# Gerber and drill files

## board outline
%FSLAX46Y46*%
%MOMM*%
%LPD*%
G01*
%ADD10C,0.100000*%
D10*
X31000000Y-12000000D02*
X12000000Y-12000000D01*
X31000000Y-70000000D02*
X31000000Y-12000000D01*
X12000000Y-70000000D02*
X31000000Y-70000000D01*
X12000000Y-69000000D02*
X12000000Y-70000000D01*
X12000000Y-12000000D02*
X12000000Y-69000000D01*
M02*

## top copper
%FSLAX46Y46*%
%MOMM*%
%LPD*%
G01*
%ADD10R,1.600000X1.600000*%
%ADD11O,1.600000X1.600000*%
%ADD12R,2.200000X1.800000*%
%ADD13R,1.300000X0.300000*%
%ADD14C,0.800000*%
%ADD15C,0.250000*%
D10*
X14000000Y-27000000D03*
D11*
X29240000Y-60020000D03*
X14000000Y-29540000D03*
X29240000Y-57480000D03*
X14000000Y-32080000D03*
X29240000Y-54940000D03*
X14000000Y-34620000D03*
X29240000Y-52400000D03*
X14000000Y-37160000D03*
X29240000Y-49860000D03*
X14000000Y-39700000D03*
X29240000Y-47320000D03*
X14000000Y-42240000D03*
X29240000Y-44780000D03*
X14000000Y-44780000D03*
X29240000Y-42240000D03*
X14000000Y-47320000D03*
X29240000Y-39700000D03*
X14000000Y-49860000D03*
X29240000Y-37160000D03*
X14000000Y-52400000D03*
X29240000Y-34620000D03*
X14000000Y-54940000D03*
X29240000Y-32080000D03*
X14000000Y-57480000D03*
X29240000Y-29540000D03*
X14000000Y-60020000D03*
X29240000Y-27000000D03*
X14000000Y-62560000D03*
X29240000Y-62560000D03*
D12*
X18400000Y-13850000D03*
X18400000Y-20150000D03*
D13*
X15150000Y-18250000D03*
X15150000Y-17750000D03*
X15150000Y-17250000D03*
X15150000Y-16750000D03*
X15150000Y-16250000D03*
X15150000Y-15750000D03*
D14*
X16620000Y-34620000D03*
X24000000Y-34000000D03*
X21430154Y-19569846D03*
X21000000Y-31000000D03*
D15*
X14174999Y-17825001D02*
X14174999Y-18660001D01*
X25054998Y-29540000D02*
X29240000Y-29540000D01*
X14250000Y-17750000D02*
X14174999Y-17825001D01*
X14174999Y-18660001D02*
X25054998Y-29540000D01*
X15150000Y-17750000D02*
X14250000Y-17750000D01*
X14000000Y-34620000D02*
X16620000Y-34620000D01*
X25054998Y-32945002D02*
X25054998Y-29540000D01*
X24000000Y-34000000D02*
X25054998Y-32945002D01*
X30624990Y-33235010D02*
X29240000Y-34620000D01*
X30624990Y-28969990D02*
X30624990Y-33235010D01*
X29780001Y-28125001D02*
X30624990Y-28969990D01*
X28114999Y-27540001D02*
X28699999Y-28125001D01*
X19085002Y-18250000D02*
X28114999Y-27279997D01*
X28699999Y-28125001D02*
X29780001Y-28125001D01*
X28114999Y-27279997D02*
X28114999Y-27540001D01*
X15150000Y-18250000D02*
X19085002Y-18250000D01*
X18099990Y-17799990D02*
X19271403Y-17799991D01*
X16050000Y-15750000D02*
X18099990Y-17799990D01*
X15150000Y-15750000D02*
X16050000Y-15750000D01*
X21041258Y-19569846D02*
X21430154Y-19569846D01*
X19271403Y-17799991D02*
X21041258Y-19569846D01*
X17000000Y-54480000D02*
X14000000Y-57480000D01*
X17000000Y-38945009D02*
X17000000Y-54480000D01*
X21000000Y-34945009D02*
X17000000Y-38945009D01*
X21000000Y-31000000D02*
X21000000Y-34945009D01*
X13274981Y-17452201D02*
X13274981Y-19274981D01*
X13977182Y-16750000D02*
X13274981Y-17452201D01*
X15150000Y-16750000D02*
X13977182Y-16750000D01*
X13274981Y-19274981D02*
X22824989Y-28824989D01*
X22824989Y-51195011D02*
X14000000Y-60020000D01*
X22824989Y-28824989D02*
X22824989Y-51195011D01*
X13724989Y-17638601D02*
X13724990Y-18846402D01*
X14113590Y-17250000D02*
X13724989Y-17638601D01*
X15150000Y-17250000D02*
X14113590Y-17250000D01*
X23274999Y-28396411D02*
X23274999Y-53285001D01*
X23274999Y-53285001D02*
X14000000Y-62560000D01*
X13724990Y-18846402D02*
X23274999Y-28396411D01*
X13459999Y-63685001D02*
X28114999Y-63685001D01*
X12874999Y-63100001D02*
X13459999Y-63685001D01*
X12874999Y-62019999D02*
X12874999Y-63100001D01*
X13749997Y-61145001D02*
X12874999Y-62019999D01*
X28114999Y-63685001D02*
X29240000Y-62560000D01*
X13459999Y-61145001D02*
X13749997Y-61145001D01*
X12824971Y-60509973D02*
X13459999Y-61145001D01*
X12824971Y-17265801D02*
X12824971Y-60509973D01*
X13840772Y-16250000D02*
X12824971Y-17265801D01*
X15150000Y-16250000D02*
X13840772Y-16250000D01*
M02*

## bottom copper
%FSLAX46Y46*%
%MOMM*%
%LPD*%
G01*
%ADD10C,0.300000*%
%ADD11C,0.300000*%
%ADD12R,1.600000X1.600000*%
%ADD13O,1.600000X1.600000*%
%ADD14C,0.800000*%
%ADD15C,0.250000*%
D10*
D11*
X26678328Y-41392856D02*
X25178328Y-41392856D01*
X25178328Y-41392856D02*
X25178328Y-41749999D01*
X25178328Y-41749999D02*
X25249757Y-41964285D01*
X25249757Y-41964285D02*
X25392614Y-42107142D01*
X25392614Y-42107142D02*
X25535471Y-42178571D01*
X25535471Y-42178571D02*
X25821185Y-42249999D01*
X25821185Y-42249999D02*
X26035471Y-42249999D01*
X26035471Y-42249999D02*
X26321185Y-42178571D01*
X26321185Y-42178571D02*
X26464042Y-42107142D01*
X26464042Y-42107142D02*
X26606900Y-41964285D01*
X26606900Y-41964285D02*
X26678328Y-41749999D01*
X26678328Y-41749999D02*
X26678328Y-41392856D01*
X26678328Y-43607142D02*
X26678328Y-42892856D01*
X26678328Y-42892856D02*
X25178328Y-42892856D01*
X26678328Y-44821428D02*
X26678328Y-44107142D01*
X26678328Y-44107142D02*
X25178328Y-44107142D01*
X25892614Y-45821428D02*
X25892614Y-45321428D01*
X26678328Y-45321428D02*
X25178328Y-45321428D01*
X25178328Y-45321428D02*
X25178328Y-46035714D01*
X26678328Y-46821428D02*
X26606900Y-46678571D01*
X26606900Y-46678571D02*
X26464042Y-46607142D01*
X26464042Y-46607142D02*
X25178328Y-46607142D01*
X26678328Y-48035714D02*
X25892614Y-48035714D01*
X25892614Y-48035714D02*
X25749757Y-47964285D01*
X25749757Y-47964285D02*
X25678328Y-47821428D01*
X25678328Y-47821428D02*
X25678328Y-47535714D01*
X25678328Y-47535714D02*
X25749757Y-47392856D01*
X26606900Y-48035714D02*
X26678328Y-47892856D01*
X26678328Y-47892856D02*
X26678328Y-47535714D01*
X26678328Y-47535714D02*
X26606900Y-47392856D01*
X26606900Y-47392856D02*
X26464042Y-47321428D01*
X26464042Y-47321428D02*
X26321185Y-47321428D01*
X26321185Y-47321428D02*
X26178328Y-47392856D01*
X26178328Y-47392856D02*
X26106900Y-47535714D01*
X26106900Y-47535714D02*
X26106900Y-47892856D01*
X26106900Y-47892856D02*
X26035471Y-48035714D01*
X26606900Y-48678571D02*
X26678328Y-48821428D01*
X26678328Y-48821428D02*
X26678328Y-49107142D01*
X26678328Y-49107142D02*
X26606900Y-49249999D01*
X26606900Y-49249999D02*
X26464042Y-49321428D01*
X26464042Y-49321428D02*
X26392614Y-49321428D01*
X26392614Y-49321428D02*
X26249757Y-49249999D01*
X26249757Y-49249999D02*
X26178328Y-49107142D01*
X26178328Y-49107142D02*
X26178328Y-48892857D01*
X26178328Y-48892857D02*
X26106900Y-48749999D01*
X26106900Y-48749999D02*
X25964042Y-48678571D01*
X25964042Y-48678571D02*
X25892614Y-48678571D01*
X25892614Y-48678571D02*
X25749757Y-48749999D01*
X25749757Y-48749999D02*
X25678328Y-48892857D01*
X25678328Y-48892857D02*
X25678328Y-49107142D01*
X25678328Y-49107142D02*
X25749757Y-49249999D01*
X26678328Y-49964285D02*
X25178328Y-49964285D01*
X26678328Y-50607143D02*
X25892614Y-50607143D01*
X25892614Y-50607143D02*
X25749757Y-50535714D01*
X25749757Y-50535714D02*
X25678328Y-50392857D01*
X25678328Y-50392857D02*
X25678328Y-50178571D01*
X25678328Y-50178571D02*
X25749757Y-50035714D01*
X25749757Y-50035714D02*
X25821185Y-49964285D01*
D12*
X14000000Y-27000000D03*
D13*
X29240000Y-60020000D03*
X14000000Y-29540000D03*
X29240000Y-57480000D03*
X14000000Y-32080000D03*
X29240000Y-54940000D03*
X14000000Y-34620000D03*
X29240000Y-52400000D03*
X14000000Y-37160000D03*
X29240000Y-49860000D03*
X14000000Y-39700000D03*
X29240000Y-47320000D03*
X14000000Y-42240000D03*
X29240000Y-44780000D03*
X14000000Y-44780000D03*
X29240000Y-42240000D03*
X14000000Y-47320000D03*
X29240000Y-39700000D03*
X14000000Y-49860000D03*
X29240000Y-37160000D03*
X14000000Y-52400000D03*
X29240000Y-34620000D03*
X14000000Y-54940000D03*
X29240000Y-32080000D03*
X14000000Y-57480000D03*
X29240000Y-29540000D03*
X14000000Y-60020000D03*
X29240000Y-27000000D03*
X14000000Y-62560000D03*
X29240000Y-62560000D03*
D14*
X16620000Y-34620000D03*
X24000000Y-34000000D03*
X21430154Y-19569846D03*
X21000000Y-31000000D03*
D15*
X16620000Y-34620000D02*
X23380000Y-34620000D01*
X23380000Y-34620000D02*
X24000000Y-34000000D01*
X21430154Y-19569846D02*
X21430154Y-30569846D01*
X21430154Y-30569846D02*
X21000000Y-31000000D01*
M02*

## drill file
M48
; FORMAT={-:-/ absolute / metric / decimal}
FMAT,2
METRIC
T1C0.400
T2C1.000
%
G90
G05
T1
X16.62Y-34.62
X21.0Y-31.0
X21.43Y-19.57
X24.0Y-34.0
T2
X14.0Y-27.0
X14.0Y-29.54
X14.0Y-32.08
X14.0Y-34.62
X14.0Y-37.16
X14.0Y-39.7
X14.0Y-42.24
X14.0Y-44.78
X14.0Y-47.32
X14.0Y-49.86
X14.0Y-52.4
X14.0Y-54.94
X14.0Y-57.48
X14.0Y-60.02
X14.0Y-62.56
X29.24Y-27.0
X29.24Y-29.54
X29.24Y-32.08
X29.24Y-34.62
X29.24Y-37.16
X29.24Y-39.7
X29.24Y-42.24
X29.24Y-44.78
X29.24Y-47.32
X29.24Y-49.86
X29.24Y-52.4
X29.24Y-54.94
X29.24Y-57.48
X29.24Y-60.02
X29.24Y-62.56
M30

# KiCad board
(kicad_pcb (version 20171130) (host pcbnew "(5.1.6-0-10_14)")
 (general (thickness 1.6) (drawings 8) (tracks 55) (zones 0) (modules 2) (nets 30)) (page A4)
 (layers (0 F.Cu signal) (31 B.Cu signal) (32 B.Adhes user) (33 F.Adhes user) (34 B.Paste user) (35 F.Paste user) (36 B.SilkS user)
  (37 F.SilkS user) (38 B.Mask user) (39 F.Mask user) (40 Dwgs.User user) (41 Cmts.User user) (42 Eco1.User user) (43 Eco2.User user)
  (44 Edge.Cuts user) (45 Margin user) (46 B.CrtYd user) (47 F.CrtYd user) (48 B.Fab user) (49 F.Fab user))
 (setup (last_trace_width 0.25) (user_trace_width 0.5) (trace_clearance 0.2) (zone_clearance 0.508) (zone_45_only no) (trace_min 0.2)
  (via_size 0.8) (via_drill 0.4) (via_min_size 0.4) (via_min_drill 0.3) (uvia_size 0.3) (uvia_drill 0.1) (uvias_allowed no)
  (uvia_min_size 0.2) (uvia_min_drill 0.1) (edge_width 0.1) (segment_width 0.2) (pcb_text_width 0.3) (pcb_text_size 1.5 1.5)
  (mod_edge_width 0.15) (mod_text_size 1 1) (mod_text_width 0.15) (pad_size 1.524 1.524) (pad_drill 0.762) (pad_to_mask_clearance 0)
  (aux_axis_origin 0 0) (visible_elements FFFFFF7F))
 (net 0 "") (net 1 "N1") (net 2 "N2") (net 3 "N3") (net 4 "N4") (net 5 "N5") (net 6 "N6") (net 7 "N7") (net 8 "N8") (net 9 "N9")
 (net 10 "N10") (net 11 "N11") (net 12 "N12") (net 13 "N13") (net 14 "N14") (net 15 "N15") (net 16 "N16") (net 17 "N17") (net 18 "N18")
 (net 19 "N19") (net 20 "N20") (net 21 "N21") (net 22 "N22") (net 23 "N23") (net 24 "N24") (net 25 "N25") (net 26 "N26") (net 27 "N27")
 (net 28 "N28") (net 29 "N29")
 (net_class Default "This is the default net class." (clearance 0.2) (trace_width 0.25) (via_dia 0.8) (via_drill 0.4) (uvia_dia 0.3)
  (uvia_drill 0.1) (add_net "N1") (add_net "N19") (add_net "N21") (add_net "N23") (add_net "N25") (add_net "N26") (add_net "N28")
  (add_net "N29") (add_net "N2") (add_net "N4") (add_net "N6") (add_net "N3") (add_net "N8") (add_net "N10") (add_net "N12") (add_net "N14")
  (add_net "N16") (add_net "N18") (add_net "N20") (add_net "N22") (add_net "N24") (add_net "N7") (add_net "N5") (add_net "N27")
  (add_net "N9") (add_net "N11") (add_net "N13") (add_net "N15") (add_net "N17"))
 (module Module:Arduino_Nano (layer F.Cu) (at 14 27)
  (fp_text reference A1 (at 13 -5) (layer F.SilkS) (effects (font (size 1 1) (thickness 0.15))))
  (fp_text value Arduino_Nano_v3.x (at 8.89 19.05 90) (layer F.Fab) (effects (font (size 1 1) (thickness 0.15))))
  (pad 1 thru_hole rect (at 0 0) (size 1.6 1.6) (drill 1) (layers *.Cu *.Mask) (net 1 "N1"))
  (pad 17 thru_hole oval (at 15.24 33.02) (size 1.6 1.6) (drill 1) (layers *.Cu *.Mask) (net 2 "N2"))
  (pad 2 thru_hole oval (at 0 2.54) (size 1.6 1.6) (drill 1) (layers *.Cu *.Mask) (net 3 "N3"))
  (pad 18 thru_hole oval (at 15.24 30.48) (size 1.6 1.6) (drill 1) (layers *.Cu *.Mask) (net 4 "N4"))
  (pad 3 thru_hole oval (at 0 5.08) (size 1.6 1.6) (drill 1) (layers *.Cu *.Mask) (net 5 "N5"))
  (pad 19 thru_hole oval (at 15.24 27.94) (size 1.6 1.6) (drill 1) (layers *.Cu *.Mask) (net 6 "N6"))
  (pad 4 thru_hole oval (at 0 7.62) (size 1.6 1.6) (drill 1) (layers *.Cu *.Mask) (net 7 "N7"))
  (pad 20 thru_hole oval (at 15.24 25.4) (size 1.6 1.6) (drill 1) (layers *.Cu *.Mask) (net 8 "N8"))
  (pad 5 thru_hole oval (at 0 10.16) (size 1.6 1.6) (drill 1) (layers *.Cu *.Mask) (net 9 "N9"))
  (pad 21 thru_hole oval (at 15.24 22.86) (size 1.6 1.6) (drill 1) (layers *.Cu *.Mask) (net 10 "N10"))
  (pad 6 thru_hole oval (at 0 12.7) (size 1.6 1.6) (drill 1) (layers *.Cu *.Mask) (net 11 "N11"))
  (pad 22 thru_hole oval (at 15.24 20.32) (size 1.6 1.6) (drill 1) (layers *.Cu *.Mask) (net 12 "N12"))
  (pad 7 thru_hole oval (at 0 15.24) (size 1.6 1.6) (drill 1) (layers *.Cu *.Mask) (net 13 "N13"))
  (pad 23 thru_hole oval (at 15.24 17.78) (size 1.6 1.6) (drill 1) (layers *.Cu *.Mask) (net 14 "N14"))
  (pad 8 thru_hole oval (at 0 17.78) (size 1.6 1.6) (drill 1) (layers *.Cu *.Mask) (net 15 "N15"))
  (pad 24 thru_hole oval (at 15.24 15.24) (size 1.6 1.6) (drill 1) (layers *.Cu *.Mask) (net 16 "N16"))
  (pad 9 thru_hole oval (at 0 20.32) (size 1.6 1.6) (drill 1) (layers *.Cu *.Mask) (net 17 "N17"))
  (pad 25 thru_hole oval (at 15.24 12.7) (size 1.6 1.6) (drill 1) (layers *.Cu *.Mask) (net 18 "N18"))
  (pad 10 thru_hole oval (at 0 22.86) (size 1.6 1.6) (drill 1) (layers *.Cu *.Mask) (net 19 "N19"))
  (pad 26 thru_hole oval (at 15.24 10.16) (size 1.6 1.6) (drill 1) (layers *.Cu *.Mask) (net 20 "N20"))
  (pad 11 thru_hole oval (at 0 25.4) (size 1.6 1.6) (drill 1) (layers *.Cu *.Mask) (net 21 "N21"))
  (pad 27 thru_hole oval (at 15.24 7.62) (size 1.6 1.6) (drill 1) (layers *.Cu *.Mask) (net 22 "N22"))
  (pad 12 thru_hole oval (at 0 27.94) (size 1.6 1.6) (drill 1) (layers *.Cu *.Mask) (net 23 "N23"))
  (pad 28 thru_hole oval (at 15.24 5.08) (size 1.6 1.6) (drill 1) (layers *.Cu *.Mask) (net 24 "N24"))
  (pad 13 thru_hole oval (at 0 30.48) (size 1.6 1.6) (drill 1) (layers *.Cu *.Mask) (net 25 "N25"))
  (pad 29 thru_hole oval (at 15.24 2.54) (size 1.6 1.6) (drill 1) (layers *.Cu *.Mask) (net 7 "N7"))
  (pad 14 thru_hole oval (at 0 33.02) (size 1.6 1.6) (drill 1) (layers *.Cu *.Mask) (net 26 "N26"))
  (pad 30 thru_hole oval (at 15.24 0) (size 1.6 1.6) (drill 1) (layers *.Cu *.Mask) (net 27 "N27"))
  (pad 15 thru_hole oval (at 0 35.56) (size 1.6 1.6) (drill 1) (layers *.Cu *.Mask) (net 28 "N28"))
  (pad 16 thru_hole oval (at 15.24 35.56) (size 1.6 1.6) (drill 1) (layers *.Cu *.Mask) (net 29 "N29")))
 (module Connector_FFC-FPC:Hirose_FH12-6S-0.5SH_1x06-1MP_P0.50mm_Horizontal (layer F.Cu) (at 17 17 90)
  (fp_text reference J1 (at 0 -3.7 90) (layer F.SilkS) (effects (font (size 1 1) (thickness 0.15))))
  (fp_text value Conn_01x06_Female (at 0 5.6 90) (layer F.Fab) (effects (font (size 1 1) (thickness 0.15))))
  (pad MP smd rect (at 3.15 1.4 90) (size 1.8 2.2) (layers F.Cu F.Paste F.Mask))
  (pad MP smd rect (at -3.15 1.4 90) (size 1.8 2.2) (layers F.Cu F.Paste F.Mask))
  (pad 1 smd rect (at -1.25 -1.85 90) (size 0.3 1.3) (layers F.Cu F.Paste F.Mask) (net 22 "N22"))
  (pad 2 smd rect (at -0.75 -1.85 90) (size 0.3 1.3) (layers F.Cu F.Paste F.Mask) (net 7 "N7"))
  (pad 3 smd rect (at -0.25 -1.85 90) (size 0.3 1.3) (layers F.Cu F.Paste F.Mask) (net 28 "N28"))
  (pad 4 smd rect (at 0.25 -1.85 90) (size 0.3 1.3) (layers F.Cu F.Paste F.Mask) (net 26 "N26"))
  (pad 5 smd rect (at 0.75 -1.85 90) (size 0.3 1.3) (layers F.Cu F.Paste F.Mask) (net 29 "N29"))
  (pad 6 smd rect (at 1.25 -1.85 90) (size 0.3 1.3) (layers F.Cu F.Paste F.Mask) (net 25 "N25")))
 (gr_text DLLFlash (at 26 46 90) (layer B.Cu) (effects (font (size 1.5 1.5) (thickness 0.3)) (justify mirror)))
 (gr_line (start 31 12) (end 12 12) (layer Edge.Cuts) (width 0.1))
 (gr_line (start 31 70) (end 31 12) (layer Edge.Cuts) (width 0.1))
 (gr_line (start 12 70) (end 31 70) (layer Edge.Cuts) (width 0.1))
 (gr_line (start 12 69) (end 12 70) (layer Edge.Cuts) (width 0.1))
 (gr_line (start 12 12) (end 12 69) (layer Edge.Cuts) (width 0.1))
 (segment (start 14.174999 17.825001) (end 14.174999 18.660001) (width 0.25) (layer F.Cu) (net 7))
 (segment (start 25.054998 29.54) (end 29.24 29.54) (width 0.25) (layer F.Cu) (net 7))
 (segment (start 14.25 17.75) (end 14.174999 17.825001) (width 0.25) (layer F.Cu) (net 7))
 (segment (start 14.174999 18.660001) (end 25.054998 29.54) (width 0.25) (layer F.Cu) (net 7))
 (segment (start 15.15 17.75) (end 14.25 17.75) (width 0.25) (layer F.Cu) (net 7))
 (segment (start 14 34.62) (end 16.62 34.62) (width 0.25) (layer F.Cu) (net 7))
 (via (at 16.62 34.62) (size 0.8) (drill 0.4) (layers F.Cu B.Cu) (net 7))
 (segment (start 16.62 34.62) (end 23.38 34.62) (width 0.25) (layer B.Cu) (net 7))
 (via (at 24 34) (size 0.8) (drill 0.4) (layers F.Cu B.Cu) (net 7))
 (segment (start 23.38 34.62) (end 24 34) (width 0.25) (layer B.Cu) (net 7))
 (segment (start 25.054998 32.945002) (end 25.054998 29.54) (width 0.25) (layer F.Cu) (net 7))
 (segment (start 24 34) (end 25.054998 32.945002) (width 0.25) (layer F.Cu) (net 7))
 (segment (start 30.62499 33.23501) (end 29.24 34.62) (width 0.25) (layer F.Cu) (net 22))
 (segment (start 30.62499 28.96999) (end 30.62499 33.23501) (width 0.25) (layer F.Cu) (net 22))
 (segment (start 29.780001 28.125001) (end 30.62499 28.96999) (width 0.25) (layer F.Cu) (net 22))
 (segment (start 28.114999 27.540001) (end 28.699999 28.125001) (width 0.25) (layer F.Cu) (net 22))
 (segment (start 19.085002 18.25) (end 28.114999 27.279997) (width 0.25) (layer F.Cu) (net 22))
 (segment (start 28.699999 28.125001) (end 29.780001 28.125001) (width 0.25) (layer F.Cu) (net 22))
 (segment (start 28.114999 27.279997) (end 28.114999 27.540001) (width 0.25) (layer F.Cu) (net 22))
 (segment (start 15.15 18.25) (end 19.085002 18.25) (width 0.25) (layer F.Cu) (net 22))
 (segment (start 18.09999 17.79999) (end 19.271403 17.799991) (width 0.25) (layer F.Cu) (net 25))
 (segment (start 16.05 15.75) (end 18.09999 17.79999) (width 0.25) (layer F.Cu) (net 25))
 (segment (start 15.15 15.75) (end 16.05 15.75) (width 0.25) (layer F.Cu) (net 25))
 (via (at 21.430154 19.569846) (size 0.8) (drill 0.4) (layers F.Cu B.Cu) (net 25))
 (segment (start 21.041258 19.569846) (end 21.430154 19.569846) (width 0.25) (layer F.Cu) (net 25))
 (segment (start 19.271403 17.799991) (end 21.041258 19.569846) (width 0.25) (layer F.Cu) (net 25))
 (segment (start 21.430154 19.569846) (end 21.430154 30.569846) (width 0.25) (layer B.Cu) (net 25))
 (via (at 21 31) (size 0.8) (drill 0.4) (layers F.Cu B.Cu) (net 25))
 (segment (start 21.430154 30.569846) (end 21 31) (width 0.25) (layer B.Cu) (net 25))
 (segment (start 17 54.48) (end 14 57.48) (width 0.25) (layer F.Cu) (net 25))
 (segment (start 17 38.945009) (end 17 54.48) (width 0.25) (layer F.Cu) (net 25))
 (segment (start 21 34.945009) (end 17 38.945009) (width 0.25) (layer F.Cu) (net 25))
 (segment (start 21 31) (end 21 34.945009) (width 0.25) (layer F.Cu) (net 25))
 (segment (start 13.274981 17.452201) (end 13.274981 19.274981) (width 0.25) (layer F.Cu) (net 26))
 (segment (start 13.977182 16.75) (end 13.274981 17.452201) (width 0.25) (layer F.Cu) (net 26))
 (segment (start 15.15 16.75) (end 13.977182 16.75) (width 0.25) (layer F.Cu) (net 26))
 (segment (start 13.274981 19.274981) (end 22.824989 28.824989) (width 0.25) (layer F.Cu) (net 26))
 (segment (start 22.824989 51.195011) (end 14 60.02) (width 0.25) (layer F.Cu) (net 26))
 (segment (start 22.824989 28.824989) (end 22.824989 51.195011) (width 0.25) (layer F.Cu) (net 26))
 (segment (start 13.724989 17.638601) (end 13.72499 18.846402) (width 0.25) (layer F.Cu) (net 28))
 (segment (start 14.11359 17.25) (end 13.724989 17.638601) (width 0.25) (layer F.Cu) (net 28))
 (segment (start 15.15 17.25) (end 14.11359 17.25) (width 0.25) (layer F.Cu) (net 28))
 (segment (start 23.274999 28.396411) (end 23.274999 53.285001) (width 0.25) (layer F.Cu) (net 28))
 (segment (start 23.274999 53.285001) (end 14 62.56) (width 0.25) (layer F.Cu) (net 28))
 (segment (start 13.72499 18.846402) (end 23.274999 28.396411) (width 0.25) (layer F.Cu) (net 28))
 (segment (start 13.459999 63.685001) (end 28.114999 63.685001) (width 0.25) (layer F.Cu) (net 29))
 (segment (start 12.874999 63.100001) (end 13.459999 63.685001) (width 0.25) (layer F.Cu) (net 29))
 (segment (start 12.874999 62.019999) (end 12.874999 63.100001) (width 0.25) (layer F.Cu) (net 29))
 (segment (start 13.749997 61.145001) (end 12.874999 62.019999) (width 0.25) (layer F.Cu) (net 29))
 (segment (start 28.114999 63.685001) (end 29.24 62.56) (width 0.25) (layer F.Cu) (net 29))
 (segment (start 13.459999 61.145001) (end 13.749997 61.145001) (width 0.25) (layer F.Cu) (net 29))
 (segment (start 12.824971 60.509973) (end 13.459999 61.145001) (width 0.25) (layer F.Cu) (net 29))
 (segment (start 12.824971 17.265801) (end 12.824971 60.509973) (width 0.25) (layer F.Cu) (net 29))
 (segment (start 13.840772 16.25) (end 12.824971 17.265801) (width 0.25) (layer F.Cu) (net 29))
 (segment (start 15.15 16.25) (end 13.840772 16.25) (width 0.25) (layer F.Cu) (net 29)))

